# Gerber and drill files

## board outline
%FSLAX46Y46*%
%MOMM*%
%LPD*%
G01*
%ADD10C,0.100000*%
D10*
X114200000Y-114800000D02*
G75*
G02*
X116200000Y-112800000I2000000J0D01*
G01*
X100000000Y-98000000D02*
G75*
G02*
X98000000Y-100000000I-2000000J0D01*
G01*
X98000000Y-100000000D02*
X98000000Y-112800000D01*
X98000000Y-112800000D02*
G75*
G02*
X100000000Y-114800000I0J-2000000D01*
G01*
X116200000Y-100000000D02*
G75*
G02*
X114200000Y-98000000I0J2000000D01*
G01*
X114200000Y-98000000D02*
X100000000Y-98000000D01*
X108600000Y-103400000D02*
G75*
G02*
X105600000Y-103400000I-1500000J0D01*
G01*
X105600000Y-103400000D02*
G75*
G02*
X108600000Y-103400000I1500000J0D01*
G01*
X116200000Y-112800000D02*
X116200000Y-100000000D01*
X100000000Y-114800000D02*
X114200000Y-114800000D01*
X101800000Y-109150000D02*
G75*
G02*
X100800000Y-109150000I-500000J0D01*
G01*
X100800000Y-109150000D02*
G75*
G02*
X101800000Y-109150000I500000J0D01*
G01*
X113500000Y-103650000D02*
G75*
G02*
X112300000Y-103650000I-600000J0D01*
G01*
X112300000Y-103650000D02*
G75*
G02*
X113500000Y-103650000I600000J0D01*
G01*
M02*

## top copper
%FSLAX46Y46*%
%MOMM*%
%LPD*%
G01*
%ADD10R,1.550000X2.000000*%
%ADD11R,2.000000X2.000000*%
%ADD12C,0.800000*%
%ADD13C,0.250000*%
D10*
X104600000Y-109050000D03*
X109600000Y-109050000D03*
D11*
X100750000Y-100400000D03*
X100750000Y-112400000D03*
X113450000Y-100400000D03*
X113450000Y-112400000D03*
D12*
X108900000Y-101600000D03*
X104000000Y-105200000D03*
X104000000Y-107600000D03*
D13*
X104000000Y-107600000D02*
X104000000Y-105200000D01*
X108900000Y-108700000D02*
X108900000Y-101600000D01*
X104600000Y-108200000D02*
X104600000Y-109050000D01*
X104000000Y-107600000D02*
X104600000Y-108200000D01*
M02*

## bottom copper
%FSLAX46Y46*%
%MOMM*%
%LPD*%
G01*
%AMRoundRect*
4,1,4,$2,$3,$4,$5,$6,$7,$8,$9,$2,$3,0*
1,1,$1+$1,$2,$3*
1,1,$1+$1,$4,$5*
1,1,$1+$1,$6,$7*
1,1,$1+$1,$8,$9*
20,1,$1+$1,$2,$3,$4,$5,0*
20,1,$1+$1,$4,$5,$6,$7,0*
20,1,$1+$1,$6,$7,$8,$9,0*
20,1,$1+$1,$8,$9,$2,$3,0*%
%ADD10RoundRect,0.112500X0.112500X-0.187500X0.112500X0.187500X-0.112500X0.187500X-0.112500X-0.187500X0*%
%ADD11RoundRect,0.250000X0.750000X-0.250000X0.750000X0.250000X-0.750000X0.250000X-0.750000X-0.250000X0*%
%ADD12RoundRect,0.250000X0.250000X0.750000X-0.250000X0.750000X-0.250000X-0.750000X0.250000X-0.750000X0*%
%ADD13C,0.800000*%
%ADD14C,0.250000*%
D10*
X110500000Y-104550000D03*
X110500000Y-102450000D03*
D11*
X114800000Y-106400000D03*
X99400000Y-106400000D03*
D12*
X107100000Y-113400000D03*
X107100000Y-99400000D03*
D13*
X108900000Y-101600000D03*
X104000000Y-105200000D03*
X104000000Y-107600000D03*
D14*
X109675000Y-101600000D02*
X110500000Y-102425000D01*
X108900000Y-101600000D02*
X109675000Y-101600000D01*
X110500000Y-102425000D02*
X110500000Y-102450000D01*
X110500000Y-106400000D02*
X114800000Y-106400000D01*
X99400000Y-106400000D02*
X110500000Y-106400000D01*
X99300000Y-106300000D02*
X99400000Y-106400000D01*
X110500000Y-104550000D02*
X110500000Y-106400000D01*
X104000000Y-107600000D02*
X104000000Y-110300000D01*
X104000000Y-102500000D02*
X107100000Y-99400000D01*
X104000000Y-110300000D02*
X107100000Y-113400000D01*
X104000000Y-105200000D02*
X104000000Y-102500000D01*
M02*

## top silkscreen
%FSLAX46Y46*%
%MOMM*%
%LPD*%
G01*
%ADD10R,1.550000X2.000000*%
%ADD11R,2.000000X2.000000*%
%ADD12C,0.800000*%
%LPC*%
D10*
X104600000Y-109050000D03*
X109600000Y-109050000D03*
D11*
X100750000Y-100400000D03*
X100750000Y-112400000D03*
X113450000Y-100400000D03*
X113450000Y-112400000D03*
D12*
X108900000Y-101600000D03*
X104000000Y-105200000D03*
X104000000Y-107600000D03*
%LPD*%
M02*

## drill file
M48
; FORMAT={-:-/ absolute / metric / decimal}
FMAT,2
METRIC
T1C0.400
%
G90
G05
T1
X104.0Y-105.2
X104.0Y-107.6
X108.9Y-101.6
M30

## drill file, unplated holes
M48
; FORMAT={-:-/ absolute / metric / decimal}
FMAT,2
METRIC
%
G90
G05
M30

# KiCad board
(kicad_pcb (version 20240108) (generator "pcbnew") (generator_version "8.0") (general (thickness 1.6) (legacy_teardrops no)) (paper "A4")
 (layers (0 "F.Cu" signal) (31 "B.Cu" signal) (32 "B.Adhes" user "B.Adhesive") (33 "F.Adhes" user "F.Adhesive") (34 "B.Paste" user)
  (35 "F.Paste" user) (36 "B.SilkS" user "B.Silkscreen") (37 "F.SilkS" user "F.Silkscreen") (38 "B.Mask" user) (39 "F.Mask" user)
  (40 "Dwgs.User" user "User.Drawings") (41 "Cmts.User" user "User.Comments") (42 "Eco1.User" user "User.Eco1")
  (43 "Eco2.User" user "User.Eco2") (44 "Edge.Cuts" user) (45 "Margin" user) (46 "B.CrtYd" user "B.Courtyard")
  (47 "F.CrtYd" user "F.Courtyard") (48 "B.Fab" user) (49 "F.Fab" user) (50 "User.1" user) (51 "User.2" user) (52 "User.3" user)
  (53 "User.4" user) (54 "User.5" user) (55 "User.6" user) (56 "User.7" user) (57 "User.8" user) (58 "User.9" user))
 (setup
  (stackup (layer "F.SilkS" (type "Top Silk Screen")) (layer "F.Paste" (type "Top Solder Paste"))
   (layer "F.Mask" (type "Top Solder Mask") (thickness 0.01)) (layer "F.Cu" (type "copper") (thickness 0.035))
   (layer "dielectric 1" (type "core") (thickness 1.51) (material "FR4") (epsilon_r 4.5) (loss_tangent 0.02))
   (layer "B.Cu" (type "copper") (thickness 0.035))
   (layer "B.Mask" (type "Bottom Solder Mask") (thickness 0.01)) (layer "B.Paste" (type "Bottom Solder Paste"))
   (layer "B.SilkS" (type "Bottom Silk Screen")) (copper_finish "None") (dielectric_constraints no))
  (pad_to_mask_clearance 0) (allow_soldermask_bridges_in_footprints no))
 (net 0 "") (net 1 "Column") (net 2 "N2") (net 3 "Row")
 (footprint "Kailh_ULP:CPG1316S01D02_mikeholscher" (layer "F.Cu") (at 107.1 106.4)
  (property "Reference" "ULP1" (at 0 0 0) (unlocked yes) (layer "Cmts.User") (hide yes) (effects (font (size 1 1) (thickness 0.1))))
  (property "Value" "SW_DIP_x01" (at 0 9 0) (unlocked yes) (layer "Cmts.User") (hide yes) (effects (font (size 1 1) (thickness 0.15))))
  (fp_circle (center -5.8 2.75) (end -5.3 2.75) (stroke (width 0.1) (type default)) (fill none) (layer "Edge.Cuts"))
  (fp_circle (center 5.8 -2.75) (end 6.4 -2.75) (stroke (width 0.1) (type default)) (fill none) (layer "Edge.Cuts"))
  (pad "1" smd rect (at -2.5 2.65) (size 1.55 2) (layers "F.Cu" "F.Paste" "F.Mask") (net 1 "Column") (thermal_bridge_angle 45))
  (pad "2" smd rect (at 2.5 2.65) (size 1.55 2) (layers "F.Cu" "F.Paste" "F.Mask") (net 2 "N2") (thermal_bridge_angle 45))
  (pad "3" smd rect (at -6.35 -6) (size 2 2) (layers "F.Cu" "F.Paste" "F.Mask") (thermal_bridge_angle 45))
  (pad "3" smd rect (at -6.35 6) (size 2 2) (layers "F.Cu" "F.Paste" "F.Mask") (thermal_bridge_angle 45))
  (pad "3" smd rect (at 6.35 -6) (size 2 2) (layers "F.Cu" "F.Paste" "F.Mask") (thermal_bridge_angle 45))
  (pad "3" smd rect (at 6.35 6) (size 2 2) (layers "F.Cu" "F.Paste" "F.Mask") (thermal_bridge_angle 45)))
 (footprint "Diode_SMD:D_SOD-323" (layer "B.Cu") (at 110.5 103.5 90)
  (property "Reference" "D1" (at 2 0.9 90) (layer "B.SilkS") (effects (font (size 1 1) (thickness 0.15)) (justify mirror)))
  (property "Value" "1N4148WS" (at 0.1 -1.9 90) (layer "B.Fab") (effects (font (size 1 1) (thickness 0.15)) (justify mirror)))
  (pad "1" smd roundrect (at -1.05 0 90) (size 0.6 0.45) (layers "B.Cu" "B.Paste" "B.Mask") (roundrect_rratio 0.25) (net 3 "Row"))
  (pad "2" smd roundrect (at 1.05 0 90) (size 0.6 0.45) (layers "B.Cu" "B.Paste" "B.Mask") (roundrect_rratio 0.25) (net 2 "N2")))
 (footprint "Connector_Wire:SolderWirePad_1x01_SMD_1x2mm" (layer "B.Cu") (at 114.8 106.4 90)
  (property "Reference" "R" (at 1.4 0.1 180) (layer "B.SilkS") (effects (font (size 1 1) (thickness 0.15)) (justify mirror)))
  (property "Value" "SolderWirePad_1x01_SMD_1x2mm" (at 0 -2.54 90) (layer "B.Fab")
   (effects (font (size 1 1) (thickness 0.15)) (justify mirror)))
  (pad "2" smd roundrect (at 0 0 90) (size 1 2) (layers "B.Cu" "B.Paste" "B.Mask") (roundrect_rratio 0.25) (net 3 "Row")))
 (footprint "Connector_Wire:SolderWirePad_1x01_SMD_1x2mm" (layer "B.Cu") (at 99.4 106.4 90)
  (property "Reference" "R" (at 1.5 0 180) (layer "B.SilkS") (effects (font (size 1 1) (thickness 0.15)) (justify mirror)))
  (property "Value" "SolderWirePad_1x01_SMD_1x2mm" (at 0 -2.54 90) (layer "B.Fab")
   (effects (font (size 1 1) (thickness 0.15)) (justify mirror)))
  (pad "1" smd roundrect (at 0 0 90) (size 1 2) (layers "B.Cu" "B.Paste" "B.Mask") (roundrect_rratio 0.25) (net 3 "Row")))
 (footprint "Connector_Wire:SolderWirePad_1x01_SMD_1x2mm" (layer "B.Cu") (at 107.1 113.4 180)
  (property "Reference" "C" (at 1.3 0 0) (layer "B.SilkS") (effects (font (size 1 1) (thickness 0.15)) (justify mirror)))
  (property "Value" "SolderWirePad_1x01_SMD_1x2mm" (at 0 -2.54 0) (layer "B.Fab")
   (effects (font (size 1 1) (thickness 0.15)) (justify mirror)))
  (pad "2" smd roundrect (at 0 0 180) (size 1 2) (layers "B.Cu" "B.Paste" "B.Mask") (roundrect_rratio 0.25) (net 1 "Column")))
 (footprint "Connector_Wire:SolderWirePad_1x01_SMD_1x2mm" (layer "B.Cu") (at 107.1 99.4 180)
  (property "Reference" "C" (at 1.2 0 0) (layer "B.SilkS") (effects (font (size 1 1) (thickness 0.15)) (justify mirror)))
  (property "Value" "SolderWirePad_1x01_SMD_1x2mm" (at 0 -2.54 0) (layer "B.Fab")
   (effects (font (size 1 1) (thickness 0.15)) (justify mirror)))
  (pad "1" smd roundrect (at 0 0 180) (size 1 2) (layers "B.Cu" "B.Paste" "B.Mask") (roundrect_rratio 0.25) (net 1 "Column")))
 (gr_arc (start 114.2 114.8) (mid 114.785786 113.385786) (end 116.2 112.8) (stroke (width 0.1) (type default)) (layer "Edge.Cuts"))
 (gr_arc (start 100 98) (mid 99.414214 99.414214) (end 98 100) (stroke (width 0.1) (type default)) (layer "Edge.Cuts"))
 (gr_line (start 98 100) (end 98 112.8) (stroke (width 0.1) (type default)) (layer "Edge.Cuts"))
 (gr_arc (start 98 112.8) (mid 99.414214 113.385786) (end 100 114.8) (stroke (width 0.1) (type default)) (layer "Edge.Cuts"))
 (gr_arc (start 116.2 100) (mid 114.785786 99.414214) (end 114.2 98) (stroke (width 0.1) (type default)) (layer "Edge.Cuts"))
 (gr_line (start 114.2 98) (end 100 98) (stroke (width 0.1) (type default)) (layer "Edge.Cuts"))
 (gr_circle (center 107.1 103.4) (end 108 104.6) (stroke (width 0.1) (type default)) (fill none) (layer "Edge.Cuts"))
 (gr_line (start 116.2 112.8) (end 116.2 100) (stroke (width 0.1) (type default)) (layer "Edge.Cuts"))
 (gr_line (start 100 114.8) (end 114.2 114.8) (stroke (width 0.1) (type default)) (layer "Edge.Cuts"))
 (segment (start 108.9 108.7) (end 108.9 101.6) (width 0.25) (layer "F.Cu") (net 2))
 (via (at 108.9 101.6) (size 0.8) (drill 0.4) (layers "F.Cu" "B.Cu") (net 2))
 (segment (start 109.675 101.6) (end 110.5 102.425) (width 0.25) (layer "B.Cu") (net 2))
 (segment (start 108.9 101.6) (end 109.675 101.6) (width 0.25) (layer "B.Cu") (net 2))
 (segment (start 110.5 102.425) (end 110.5 102.45) (width 0.25) (layer "B.Cu") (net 2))
 (segment (start 110.5 106.4) (end 114.8 106.4) (width 0.25) (layer "B.Cu") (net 3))
 (segment (start 99.4 106.4) (end 110.5 106.4) (width 0.25) (layer "B.Cu") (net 3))
 (segment (start 99.3 106.3) (end 99.4 106.4) (width 0.25) (layer "B.Cu") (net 3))
 (segment (start 110.5 104.55) (end 110.5 106.4) (width 0.25) (layer "B.Cu") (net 3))
 (segment (start 104 107.6) (end 104.6 108.2) (width 0.25) (layer "F.Cu") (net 1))
 (segment (start 104 107.6) (end 104 105.2) (width 0.25) (layer "F.Cu") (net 1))
 (segment (start 104.6 108.2) (end 104.6 109.05) (width 0.25) (layer "F.Cu") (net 1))
 (via (at 104 105.2) (size 0.8) (drill 0.4) (layers "F.Cu" "B.Cu") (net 1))
 (via (at 104 107.6) (size 0.8) (drill 0.4) (layers "F.Cu" "B.Cu") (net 1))
 (segment (start 104 107.6) (end 104 110.3) (width 0.25) (layer "B.Cu") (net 1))
 (segment (start 104 102.5) (end 107.1 99.4) (width 0.25) (layer "B.Cu") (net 1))
 (segment (start 104 110.3) (end 107.1 113.4) (width 0.25) (layer "B.Cu") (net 1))
 (segment (start 104 105.2) (end 104 102.5) (width 0.25) (layer "B.Cu") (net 1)))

